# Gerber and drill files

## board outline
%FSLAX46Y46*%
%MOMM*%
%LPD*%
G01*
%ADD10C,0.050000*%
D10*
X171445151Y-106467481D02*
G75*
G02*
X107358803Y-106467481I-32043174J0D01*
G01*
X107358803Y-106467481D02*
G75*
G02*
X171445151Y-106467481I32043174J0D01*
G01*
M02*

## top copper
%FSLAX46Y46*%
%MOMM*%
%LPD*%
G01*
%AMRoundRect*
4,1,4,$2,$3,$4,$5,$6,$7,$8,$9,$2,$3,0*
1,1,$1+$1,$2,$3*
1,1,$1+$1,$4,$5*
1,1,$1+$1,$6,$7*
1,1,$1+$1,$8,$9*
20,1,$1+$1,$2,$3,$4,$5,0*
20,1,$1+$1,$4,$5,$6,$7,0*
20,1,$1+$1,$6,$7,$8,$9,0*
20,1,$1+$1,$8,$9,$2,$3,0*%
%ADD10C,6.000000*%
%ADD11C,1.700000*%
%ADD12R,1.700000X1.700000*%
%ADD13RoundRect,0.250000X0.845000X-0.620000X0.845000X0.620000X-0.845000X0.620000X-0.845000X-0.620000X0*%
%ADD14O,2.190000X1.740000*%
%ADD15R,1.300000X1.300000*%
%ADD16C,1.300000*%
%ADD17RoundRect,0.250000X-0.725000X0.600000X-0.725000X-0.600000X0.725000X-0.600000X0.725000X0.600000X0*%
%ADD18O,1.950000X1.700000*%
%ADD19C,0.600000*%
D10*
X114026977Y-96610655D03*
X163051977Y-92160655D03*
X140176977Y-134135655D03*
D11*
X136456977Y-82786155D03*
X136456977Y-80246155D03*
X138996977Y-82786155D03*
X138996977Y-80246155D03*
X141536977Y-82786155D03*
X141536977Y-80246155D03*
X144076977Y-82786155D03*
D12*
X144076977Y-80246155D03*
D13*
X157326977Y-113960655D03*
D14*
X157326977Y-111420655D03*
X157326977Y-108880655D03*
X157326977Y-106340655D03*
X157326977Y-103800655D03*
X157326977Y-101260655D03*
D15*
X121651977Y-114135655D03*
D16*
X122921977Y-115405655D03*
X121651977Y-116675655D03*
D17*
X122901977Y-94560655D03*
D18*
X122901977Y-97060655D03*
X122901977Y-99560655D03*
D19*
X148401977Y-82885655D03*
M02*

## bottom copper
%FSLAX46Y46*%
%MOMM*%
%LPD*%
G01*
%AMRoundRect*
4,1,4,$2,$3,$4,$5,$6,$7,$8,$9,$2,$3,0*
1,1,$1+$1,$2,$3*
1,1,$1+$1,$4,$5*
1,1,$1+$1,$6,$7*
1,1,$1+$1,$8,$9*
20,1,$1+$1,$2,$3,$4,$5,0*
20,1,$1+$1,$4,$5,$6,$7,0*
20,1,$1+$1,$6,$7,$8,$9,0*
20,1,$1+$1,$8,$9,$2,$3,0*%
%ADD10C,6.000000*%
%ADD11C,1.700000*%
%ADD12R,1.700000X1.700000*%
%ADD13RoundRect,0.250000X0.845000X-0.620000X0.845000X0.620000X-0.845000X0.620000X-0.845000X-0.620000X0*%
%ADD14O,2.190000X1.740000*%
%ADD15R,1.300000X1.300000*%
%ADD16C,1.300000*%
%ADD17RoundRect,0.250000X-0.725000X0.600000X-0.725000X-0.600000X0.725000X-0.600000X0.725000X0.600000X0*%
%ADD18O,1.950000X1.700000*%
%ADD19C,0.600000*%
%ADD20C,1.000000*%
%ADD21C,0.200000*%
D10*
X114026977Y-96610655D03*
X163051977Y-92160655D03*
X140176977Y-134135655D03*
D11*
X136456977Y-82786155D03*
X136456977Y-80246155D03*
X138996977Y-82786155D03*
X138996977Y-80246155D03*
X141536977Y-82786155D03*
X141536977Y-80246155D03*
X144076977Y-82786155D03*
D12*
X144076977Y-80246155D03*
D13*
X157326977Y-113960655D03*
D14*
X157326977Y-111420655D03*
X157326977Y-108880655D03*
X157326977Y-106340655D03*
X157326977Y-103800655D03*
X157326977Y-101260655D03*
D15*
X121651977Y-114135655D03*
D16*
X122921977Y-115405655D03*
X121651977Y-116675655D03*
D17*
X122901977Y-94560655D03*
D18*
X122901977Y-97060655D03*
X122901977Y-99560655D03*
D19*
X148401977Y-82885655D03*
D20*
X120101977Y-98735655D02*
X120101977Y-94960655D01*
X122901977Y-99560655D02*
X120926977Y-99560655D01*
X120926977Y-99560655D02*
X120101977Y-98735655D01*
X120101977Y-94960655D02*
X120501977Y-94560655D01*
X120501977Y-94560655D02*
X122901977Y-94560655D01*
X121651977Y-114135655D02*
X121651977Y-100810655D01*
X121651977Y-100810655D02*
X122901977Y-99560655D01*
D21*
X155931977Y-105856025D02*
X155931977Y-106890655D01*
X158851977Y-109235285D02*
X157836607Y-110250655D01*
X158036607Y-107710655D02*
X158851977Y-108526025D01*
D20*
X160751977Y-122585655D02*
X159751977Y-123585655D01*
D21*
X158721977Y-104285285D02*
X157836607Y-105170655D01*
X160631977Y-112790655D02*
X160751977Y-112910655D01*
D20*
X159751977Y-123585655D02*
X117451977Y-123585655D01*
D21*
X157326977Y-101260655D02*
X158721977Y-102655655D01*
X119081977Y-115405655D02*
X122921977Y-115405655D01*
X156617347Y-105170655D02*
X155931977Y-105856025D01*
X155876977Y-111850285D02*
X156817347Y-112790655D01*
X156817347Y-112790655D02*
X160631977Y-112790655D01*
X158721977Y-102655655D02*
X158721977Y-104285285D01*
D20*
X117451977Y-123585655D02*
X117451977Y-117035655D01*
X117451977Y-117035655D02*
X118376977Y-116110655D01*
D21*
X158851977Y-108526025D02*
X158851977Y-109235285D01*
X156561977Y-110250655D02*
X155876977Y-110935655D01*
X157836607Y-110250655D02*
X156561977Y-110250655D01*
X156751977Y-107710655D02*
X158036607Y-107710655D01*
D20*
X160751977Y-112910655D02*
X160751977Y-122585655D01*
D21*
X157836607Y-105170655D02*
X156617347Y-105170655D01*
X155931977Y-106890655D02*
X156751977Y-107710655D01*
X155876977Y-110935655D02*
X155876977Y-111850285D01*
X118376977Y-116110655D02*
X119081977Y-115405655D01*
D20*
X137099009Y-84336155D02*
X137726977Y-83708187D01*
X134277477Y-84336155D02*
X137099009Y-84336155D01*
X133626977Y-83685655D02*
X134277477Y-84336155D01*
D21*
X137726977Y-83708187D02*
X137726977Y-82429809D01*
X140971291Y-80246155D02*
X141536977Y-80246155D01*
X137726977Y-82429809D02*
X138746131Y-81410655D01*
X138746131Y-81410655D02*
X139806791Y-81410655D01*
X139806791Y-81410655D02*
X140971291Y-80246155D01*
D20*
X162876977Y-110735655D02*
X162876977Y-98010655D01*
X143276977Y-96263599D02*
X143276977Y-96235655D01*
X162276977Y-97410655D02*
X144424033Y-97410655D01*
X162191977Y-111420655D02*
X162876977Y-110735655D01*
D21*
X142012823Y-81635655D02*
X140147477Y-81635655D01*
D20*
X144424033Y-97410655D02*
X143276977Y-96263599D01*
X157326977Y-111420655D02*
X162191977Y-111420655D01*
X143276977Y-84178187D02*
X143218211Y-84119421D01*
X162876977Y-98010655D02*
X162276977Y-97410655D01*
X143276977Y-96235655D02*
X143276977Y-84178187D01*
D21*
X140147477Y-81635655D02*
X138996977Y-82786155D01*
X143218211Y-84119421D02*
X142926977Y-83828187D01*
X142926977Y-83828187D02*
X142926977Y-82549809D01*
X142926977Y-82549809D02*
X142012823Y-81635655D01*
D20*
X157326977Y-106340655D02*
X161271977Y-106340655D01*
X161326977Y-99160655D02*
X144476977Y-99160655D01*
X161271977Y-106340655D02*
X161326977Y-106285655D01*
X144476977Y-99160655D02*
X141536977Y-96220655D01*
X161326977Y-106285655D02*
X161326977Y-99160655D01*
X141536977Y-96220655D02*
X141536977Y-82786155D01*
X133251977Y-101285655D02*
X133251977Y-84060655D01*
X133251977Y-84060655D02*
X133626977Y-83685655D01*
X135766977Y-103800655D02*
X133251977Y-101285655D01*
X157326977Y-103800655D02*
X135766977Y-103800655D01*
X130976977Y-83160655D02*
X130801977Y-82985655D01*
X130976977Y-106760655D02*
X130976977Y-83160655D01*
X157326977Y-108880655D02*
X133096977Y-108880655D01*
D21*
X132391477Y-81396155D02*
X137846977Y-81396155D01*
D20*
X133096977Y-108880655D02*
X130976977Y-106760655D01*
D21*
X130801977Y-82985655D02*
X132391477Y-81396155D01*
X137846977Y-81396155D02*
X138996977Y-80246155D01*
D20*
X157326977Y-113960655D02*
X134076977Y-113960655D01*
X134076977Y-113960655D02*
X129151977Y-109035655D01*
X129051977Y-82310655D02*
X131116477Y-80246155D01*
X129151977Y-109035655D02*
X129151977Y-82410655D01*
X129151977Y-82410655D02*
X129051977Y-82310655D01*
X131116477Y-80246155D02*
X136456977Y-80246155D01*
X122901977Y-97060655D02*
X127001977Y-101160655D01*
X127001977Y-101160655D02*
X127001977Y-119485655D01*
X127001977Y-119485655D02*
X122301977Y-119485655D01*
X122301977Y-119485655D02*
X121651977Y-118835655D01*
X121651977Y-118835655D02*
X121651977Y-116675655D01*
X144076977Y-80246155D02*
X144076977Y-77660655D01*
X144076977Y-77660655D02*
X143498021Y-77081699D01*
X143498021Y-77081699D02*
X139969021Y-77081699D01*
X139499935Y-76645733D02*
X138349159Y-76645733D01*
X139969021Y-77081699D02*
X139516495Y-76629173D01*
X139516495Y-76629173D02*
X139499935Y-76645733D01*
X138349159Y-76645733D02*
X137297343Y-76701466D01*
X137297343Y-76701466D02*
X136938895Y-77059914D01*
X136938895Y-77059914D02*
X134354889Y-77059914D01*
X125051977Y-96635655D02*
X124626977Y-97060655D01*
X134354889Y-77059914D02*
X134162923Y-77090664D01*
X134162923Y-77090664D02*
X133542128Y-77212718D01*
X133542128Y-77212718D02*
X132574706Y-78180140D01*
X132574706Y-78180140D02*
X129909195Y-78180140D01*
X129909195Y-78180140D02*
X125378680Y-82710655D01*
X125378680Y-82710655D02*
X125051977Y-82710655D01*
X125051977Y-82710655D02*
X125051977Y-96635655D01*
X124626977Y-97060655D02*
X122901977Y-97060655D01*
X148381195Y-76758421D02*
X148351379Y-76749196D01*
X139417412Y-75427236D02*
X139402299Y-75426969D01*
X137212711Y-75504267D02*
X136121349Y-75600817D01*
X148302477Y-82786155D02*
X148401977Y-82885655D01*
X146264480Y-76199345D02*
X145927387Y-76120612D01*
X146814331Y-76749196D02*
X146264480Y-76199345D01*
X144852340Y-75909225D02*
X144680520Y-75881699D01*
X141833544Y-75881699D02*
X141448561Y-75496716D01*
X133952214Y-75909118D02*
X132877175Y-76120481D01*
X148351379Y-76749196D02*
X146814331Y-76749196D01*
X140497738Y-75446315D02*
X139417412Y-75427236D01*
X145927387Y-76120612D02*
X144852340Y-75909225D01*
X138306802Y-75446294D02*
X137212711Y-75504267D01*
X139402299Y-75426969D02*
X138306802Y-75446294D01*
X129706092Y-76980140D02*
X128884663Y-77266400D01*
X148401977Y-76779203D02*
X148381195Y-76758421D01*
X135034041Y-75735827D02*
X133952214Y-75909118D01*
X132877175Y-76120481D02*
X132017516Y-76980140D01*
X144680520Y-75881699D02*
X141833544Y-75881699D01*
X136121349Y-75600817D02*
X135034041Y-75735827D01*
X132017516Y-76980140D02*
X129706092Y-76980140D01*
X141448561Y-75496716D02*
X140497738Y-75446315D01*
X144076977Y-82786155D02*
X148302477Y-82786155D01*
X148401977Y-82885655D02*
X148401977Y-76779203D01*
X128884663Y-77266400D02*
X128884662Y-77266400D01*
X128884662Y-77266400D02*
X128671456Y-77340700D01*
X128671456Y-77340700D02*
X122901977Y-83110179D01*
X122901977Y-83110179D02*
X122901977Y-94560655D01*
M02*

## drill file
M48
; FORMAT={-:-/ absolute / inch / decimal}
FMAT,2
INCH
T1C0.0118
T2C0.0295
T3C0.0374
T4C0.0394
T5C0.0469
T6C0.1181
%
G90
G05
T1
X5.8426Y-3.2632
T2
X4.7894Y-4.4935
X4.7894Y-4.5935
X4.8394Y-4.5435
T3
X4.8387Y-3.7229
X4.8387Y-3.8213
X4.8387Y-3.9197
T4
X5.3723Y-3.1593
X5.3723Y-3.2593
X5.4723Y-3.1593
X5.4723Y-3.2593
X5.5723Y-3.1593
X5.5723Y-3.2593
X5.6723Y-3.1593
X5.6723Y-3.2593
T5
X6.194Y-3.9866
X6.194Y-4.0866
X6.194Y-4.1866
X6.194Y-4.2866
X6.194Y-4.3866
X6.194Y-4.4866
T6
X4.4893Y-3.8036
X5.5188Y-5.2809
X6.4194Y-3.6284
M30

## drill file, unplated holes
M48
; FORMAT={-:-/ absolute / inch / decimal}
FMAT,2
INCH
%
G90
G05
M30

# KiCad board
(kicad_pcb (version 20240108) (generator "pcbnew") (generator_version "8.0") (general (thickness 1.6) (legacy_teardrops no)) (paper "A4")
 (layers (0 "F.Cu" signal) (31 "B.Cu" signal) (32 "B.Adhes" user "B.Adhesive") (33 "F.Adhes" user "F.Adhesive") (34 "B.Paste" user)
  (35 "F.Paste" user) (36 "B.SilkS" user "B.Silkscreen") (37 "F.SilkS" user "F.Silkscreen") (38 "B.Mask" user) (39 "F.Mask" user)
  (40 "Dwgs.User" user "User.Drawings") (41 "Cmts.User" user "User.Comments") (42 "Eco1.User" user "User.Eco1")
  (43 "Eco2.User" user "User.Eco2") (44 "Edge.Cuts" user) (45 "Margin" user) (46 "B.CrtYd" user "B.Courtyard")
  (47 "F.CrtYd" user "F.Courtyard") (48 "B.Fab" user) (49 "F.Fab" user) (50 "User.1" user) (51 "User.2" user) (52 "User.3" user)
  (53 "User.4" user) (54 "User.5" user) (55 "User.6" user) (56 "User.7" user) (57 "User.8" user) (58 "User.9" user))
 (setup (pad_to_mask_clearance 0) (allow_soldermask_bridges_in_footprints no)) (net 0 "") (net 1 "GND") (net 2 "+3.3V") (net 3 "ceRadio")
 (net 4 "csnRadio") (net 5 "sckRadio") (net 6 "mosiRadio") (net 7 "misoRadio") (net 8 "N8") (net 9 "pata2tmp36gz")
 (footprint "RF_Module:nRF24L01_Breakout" (layer "F.Cu") (at 144.076977 80.246155 -90)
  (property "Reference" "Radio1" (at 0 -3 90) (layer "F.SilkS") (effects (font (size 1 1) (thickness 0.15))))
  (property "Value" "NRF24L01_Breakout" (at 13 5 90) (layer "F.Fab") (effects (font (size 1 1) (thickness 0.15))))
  (pad "1" thru_hole rect (at 0 0 270) (size 1.7 1.7) (drill 1) (layers "*.Cu" "*.Mask") (remove_unused_layers no) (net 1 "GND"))
  (pad "2" thru_hole circle (at 2.54 0 270) (size 1.7 1.7) (drill 1) (layers "*.Cu" "*.Mask") (remove_unused_layers no) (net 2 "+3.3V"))
  (pad "3" thru_hole circle (at 0 2.54 270) (size 1.7 1.7) (drill 1) (layers "*.Cu" "*.Mask") (remove_unused_layers no) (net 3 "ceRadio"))
  (pad "4" thru_hole circle (at 2.54 2.54 270) (size 1.7 1.7) (drill 1) (layers "*.Cu" "*.Mask") (remove_unused_layers no)
   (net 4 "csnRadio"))
  (pad "5" thru_hole circle (at 0 5.08 270) (size 1.7 1.7) (drill 1) (layers "*.Cu" "*.Mask") (remove_unused_layers no) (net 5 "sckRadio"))
  (pad "6" thru_hole circle (at 2.54 5.08 270) (size 1.7 1.7) (drill 1) (layers "*.Cu" "*.Mask") (remove_unused_layers no)
   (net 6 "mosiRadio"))
  (pad "7" thru_hole circle (at 0 7.62 270) (size 1.7 1.7) (drill 1) (layers "*.Cu" "*.Mask") (remove_unused_layers no) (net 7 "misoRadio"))
  (pad "8" thru_hole circle (at 2.54 7.62 270) (size 1.7 1.7) (drill 1) (layers "*.Cu" "*.Mask") (remove_unused_layers no) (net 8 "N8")))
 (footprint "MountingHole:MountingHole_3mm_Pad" (layer "F.Cu") (at 163.051977 92.160655)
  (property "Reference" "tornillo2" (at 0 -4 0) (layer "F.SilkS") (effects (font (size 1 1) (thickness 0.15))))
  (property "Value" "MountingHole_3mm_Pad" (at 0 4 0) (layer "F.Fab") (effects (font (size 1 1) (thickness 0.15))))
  (pad "2" thru_hole circle (at 0 0) (size 6 6) (drill 3) (layers "*.Cu" "*.Mask") (remove_unused_layers no)))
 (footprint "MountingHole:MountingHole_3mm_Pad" (layer "F.Cu") (at 114.026977 96.610655)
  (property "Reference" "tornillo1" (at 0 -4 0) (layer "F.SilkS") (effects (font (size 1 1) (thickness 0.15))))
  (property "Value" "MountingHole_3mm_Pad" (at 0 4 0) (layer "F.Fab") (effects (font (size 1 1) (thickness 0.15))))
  (pad "1" thru_hole circle (at 0 0) (size 6 6) (drill 3) (layers "*.Cu" "*.Mask") (remove_unused_layers no)))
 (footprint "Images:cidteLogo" (layer "F.Cu") (at 139.276977 106.160655 90)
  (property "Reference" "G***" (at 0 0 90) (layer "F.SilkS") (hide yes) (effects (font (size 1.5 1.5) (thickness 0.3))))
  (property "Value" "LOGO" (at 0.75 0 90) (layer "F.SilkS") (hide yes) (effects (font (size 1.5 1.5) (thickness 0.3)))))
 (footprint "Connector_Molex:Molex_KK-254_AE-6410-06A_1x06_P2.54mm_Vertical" (layer "F.Cu") (at 157.326977 113.960655 90)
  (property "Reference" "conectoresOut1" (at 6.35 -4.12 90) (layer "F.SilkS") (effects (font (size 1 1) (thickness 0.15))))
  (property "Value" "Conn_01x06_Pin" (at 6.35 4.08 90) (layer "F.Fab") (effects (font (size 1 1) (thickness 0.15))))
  (pad "1" thru_hole roundrect (at 0 0 90) (size 1.74 2.19) (drill 1.19) (layers "*.Cu" "*.Mask") (remove_unused_layers no)
   (roundrect_rratio 0.143678) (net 7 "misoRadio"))
  (pad "2" thru_hole oval (at 2.54 0 90) (size 1.74 2.19) (drill 1.19) (layers "*.Cu" "*.Mask") (remove_unused_layers no)
   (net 6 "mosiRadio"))
  (pad "3" thru_hole oval (at 5.08 0 90) (size 1.74 2.19) (drill 1.19) (layers "*.Cu" "*.Mask") (remove_unused_layers no) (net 5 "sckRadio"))
  (pad "4" thru_hole oval (at 7.62 0 90) (size 1.74 2.19) (drill 1.19) (layers "*.Cu" "*.Mask") (remove_unused_layers no) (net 4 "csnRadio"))
  (pad "5" thru_hole oval (at 10.16 0 90) (size 1.74 2.19) (drill 1.19) (layers "*.Cu" "*.Mask") (remove_unused_layers no) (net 3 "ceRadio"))
  (pad "6" thru_hole oval (at 12.7 0 90) (size 1.74 2.19) (drill 1.19) (layers "*.Cu" "*.Mask") (remove_unused_layers no)
   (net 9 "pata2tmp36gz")))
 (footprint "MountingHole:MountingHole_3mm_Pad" (layer "F.Cu") (at 140.176977 134.135655)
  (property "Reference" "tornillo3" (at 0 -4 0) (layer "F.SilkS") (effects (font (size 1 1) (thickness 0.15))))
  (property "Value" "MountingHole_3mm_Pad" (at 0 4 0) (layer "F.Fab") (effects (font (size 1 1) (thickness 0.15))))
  (pad "3" thru_hole circle (at 0 0) (size 6 6) (drill 3) (layers "*.Cu" "*.Mask") (remove_unused_layers no)))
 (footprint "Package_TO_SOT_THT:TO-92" (layer "F.Cu") (at 121.651977 114.135655 -90)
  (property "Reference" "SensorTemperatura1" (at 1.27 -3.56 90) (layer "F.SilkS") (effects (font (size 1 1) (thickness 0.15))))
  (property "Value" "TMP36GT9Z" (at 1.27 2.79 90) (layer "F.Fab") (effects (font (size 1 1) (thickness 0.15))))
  (pad "1" thru_hole rect (at 0 0 270) (size 1.3 1.3) (drill 0.75) (layers "*.Cu" "*.Mask") (remove_unused_layers no) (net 2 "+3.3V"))
  (pad "2" thru_hole circle (at 1.27 -1.27 270) (size 1.3 1.3) (drill 0.75) (layers "*.Cu" "*.Mask") (remove_unused_layers no)
   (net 9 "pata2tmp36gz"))
  (pad "3" thru_hole circle (at 2.54 0 270) (size 1.3 1.3) (drill 0.75) (layers "*.Cu" "*.Mask") (remove_unused_layers no) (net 1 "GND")))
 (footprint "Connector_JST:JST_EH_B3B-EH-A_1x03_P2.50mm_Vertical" (layer "F.Cu") (at 122.901977 94.560655 -90)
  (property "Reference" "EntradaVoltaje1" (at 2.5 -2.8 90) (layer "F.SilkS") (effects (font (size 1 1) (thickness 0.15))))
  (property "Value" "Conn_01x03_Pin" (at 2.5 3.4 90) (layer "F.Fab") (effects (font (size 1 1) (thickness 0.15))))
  (pad "1" thru_hole roundrect (at 0 0 270) (size 1.7 1.95) (drill 0.95) (layers "*.Cu" "*.Mask") (remove_unused_layers no)
   (roundrect_rratio 0.147059) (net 2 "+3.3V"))
  (pad "2" thru_hole oval (at 2.5 0 270) (size 1.7 1.95) (drill 0.95) (layers "*.Cu" "*.Mask") (remove_unused_layers no) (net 1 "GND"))
  (pad "3" thru_hole oval (at 5 0 270) (size 1.7 1.95) (drill 0.95) (layers "*.Cu" "*.Mask") (remove_unused_layers no) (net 2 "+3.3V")))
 (gr_circle (center 139.401977 106.467481) (end 161.451977 129.717481) (stroke (width 0.05) (type default)) (fill none) (layer "Edge.Cuts"))
 (segment (start 137.099009 84.336155) (end 137.726977 83.708187) (width 1) (layer "B.Cu") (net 3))
 (segment (start 133.251977 84.060655) (end 133.626977 83.685655) (width 1) (layer "B.Cu") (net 3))
 (segment (start 137.726977 83.708187) (end 137.726977 82.429809) (width 0.2) (layer "B.Cu") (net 3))
 (segment (start 133.251977 101.285655) (end 133.251977 84.060655) (width 1) (layer "B.Cu") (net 3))
 (segment (start 157.326977 103.800655) (end 135.766977 103.800655) (width 1) (layer "B.Cu") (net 3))
 (segment (start 140.971291 80.246155) (end 141.536977 80.246155) (width 0.2) (layer "B.Cu") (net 3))
 (segment (start 135.766977 103.800655) (end 133.251977 101.285655) (width 1) (layer "B.Cu") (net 3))
 (segment (start 133.626977 83.685655) (end 134.277477 84.336155) (width 1) (layer "B.Cu") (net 3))
 (segment (start 138.746131 81.410655) (end 139.806791 81.410655) (width 0.2) (layer "B.Cu") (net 3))
 (segment (start 134.277477 84.336155) (end 137.099009 84.336155) (width 1) (layer "B.Cu") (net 3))
 (segment (start 137.726977 82.429809) (end 138.746131 81.410655) (width 0.2) (layer "B.Cu") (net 3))
 (segment (start 139.806791 81.410655) (end 140.971291 80.246155) (width 0.2) (layer "B.Cu") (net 3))
 (segment (start 141.536977 96.220655) (end 141.536977 82.786155) (width 1) (layer "B.Cu") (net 4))
 (segment (start 161.271977 106.340655) (end 161.326977 106.285655) (width 1) (layer "B.Cu") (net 4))
 (segment (start 157.326977 106.340655) (end 161.271977 106.340655) (width 1) (layer "B.Cu") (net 4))
 (segment (start 144.476977 99.160655) (end 141.536977 96.220655) (width 1) (layer "B.Cu") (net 4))
 (segment (start 161.326977 106.285655) (end 161.326977 99.160655) (width 1) (layer "B.Cu") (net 4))
 (segment (start 161.326977 99.160655) (end 144.476977 99.160655) (width 1) (layer "B.Cu") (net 4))
 (segment (start 130.976977 106.760655) (end 130.976977 83.160655) (width 1) (layer "B.Cu") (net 5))
 (segment (start 130.801977 82.985655) (end 132.391477 81.396155) (width 0.2) (layer "B.Cu") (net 5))
 (segment (start 133.096977 108.880655) (end 130.976977 106.760655) (width 1) (layer "B.Cu") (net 5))
 (segment (start 137.846977 81.396155) (end 138.996977 80.246155) (width 0.2) (layer "B.Cu") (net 5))
 (segment (start 132.391477 81.396155) (end 137.846977 81.396155) (width 0.2) (layer "B.Cu") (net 5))
 (segment (start 157.326977 108.880655) (end 133.096977 108.880655) (width 1) (layer "B.Cu") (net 5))
 (segment (start 130.976977 83.160655) (end 130.801977 82.985655) (width 1) (layer "B.Cu") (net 5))
 (segment (start 140.147477 81.635655) (end 138.996977 82.786155) (width 0.2) (layer "B.Cu") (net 6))
 (segment (start 142.926977 82.549809) (end 142.012823 81.635655) (width 0.2) (layer "B.Cu") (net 6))
 (segment (start 143.276977 84.178187) (end 143.218211 84.119421) (width 1) (layer "B.Cu") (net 6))
 (segment (start 143.218211 84.119421) (end 142.926977 83.828187) (width 0.2) (layer "B.Cu") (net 6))
 (segment (start 143.276977 96.235655) (end 143.276977 84.178187) (width 1) (layer "B.Cu") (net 6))
 (segment (start 157.326977 111.420655) (end 162.191977 111.420655) (width 1) (layer "B.Cu") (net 6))
 (segment (start 162.191977 111.420655) (end 162.876977 110.735655) (width 1) (layer "B.Cu") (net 6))
 (segment (start 162.276977 97.410655) (end 144.424033 97.410655) (width 1) (layer "B.Cu") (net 6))
 (segment (start 162.876977 110.735655) (end 162.876977 98.010655) (width 1) (layer "B.Cu") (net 6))
 (segment (start 162.876977 98.010655) (end 162.276977 97.410655) (width 1) (layer "B.Cu") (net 6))
 (segment (start 142.012823 81.635655) (end 140.147477 81.635655) (width 0.2) (layer "B.Cu") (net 6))
 (segment (start 144.424033 97.410655) (end 143.276977 96.263599) (width 1) (layer "B.Cu") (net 6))
 (segment (start 143.276977 96.263599) (end 143.276977 96.235655) (width 1) (layer "B.Cu") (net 6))
 (segment (start 142.926977 83.828187) (end 142.926977 82.549809) (width 0.2) (layer "B.Cu") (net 6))
 (segment (start 129.151977 109.035655) (end 129.151977 82.410655) (width 1) (layer "B.Cu") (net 7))
 (segment (start 129.051977 82.310655) (end 131.116477 80.246155) (width 1) (layer "B.Cu") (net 7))
 (segment (start 129.151977 82.410655) (end 129.051977 82.310655) (width 1) (layer "B.Cu") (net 7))
 (segment (start 131.116477 80.246155) (end 136.456977 80.246155) (width 1) (layer "B.Cu") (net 7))
 (segment (start 134.076977 113.960655) (end 129.151977 109.035655) (width 1) (layer "B.Cu") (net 7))
 (segment (start 157.326977 113.960655) (end 134.076977 113.960655) (width 1) (layer "B.Cu") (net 7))
 (segment (start 160.751977 122.585655) (end 159.751977 123.585655) (width 1) (layer "B.Cu") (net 9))
 (segment (start 160.631977 112.790655) (end 160.751977 112.910655) (width 0.2) (layer "B.Cu") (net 9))
 (segment (start 160.751977 112.910655) (end 160.751977 122.585655) (width 1) (layer "B.Cu") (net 9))
 (segment (start 155.876977 110.935655) (end 155.876977 111.850285) (width 0.2) (layer "B.Cu") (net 9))
 (segment (start 155.931977 106.890655) (end 156.751977 107.710655) (width 0.2) (layer "B.Cu") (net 9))
 (segment (start 156.751977 107.710655) (end 158.036607 107.710655) (width 0.2) (layer "B.Cu") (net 9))
 (segment (start 159.751977 123.585655) (end 117.451977 123.585655) (width 1) (layer "B.Cu") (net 9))
 (segment (start 158.721977 102.655655) (end 158.721977 104.285285) (width 0.2) (layer "B.Cu") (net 9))
 (segment (start 158.036607 107.710655) (end 158.851977 108.526025) (width 0.2) (layer "B.Cu") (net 9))
 (segment (start 157.836607 105.170655) (end 156.617347 105.170655) (width 0.2) (layer "B.Cu") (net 9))
 (segment (start 155.876977 111.850285) (end 156.817347 112.790655) (width 0.2) (layer "B.Cu") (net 9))
 (segment (start 158.851977 109.235285) (end 157.836607 110.250655) (width 0.2) (layer "B.Cu") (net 9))
 (segment (start 156.817347 112.790655) (end 160.631977 112.790655) (width 0.2) (layer "B.Cu") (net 9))
 (segment (start 158.851977 108.526025) (end 158.851977 109.235285) (width 0.2) (layer "B.Cu") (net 9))
 (segment (start 117.451977 117.035655) (end 118.376977 116.110655) (width 1) (layer "B.Cu") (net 9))
 (segment (start 156.561977 110.250655) (end 155.876977 110.935655) (width 0.2) (layer "B.Cu") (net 9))
 (segment (start 158.721977 104.285285) (end 157.836607 105.170655) (width 0.2) (layer "B.Cu") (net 9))
 (segment (start 118.376977 116.110655) (end 119.081977 115.405655) (width 0.2) (layer "B.Cu") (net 9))
 (segment (start 155.931977 105.856025) (end 155.931977 106.890655) (width 0.2) (layer "B.Cu") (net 9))
 (segment (start 117.451977 123.585655) (end 117.451977 117.035655) (width 1) (layer "B.Cu") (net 9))
 (segment (start 157.326977 101.260655) (end 158.721977 102.655655) (width 0.2) (layer "B.Cu") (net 9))
 (segment (start 156.617347 105.170655) (end 155.931977 105.856025) (width 0.2) (layer "B.Cu") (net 9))
 (segment (start 157.836607 110.250655) (end 156.561977 110.250655) (width 0.2) (layer "B.Cu") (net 9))
 (segment (start 119.081977 115.405655) (end 122.921977 115.405655) (width 0.2) (layer "B.Cu") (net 9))
 (via (at 148.401977 82.885655) (size 0.6) (drill 0.3) (layers "F.Cu" "B.Cu") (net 2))
 (segment (start 144.85234 75.909225) (end 144.68052 75.881699) (width 1) (layer "B.Cu") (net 2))
 (segment (start 133.952214 75.909118) (end 132.877175 76.120481) (width 1) (layer "B.Cu") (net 2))
 (segment (start 122.901977 99.560655) (end 120.926977 99.560655) (width 1) (layer "B.Cu") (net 2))
 (segment (start 120.926977 99.560655) (end 120.101977 98.735655) (width 1) (layer "B.Cu") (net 2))
 (segment (start 148.381195 76.758421) (end 148.351379 76.749196) (width 1) (layer "B.Cu") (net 2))
 (segment (start 129.706092 76.98014) (end 128.884663 77.2664) (width 1) (layer "B.Cu") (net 2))
 (segment (start 120.101977 98.735655) (end 120.101977 94.960655) (width 1) (layer "B.Cu") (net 2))
 (segment (start 137.212711 75.504267) (end 136.121349 75.600817) (width 1) (layer "B.Cu") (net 2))
 (segment (start 144.68052 75.881699) (end 141.833544 75.881699) (width 1) (layer "B.Cu") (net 2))
 (segment (start 148.302477 82.786155) (end 148.401977 82.885655) (width 1) (layer "B.Cu") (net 2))
 (segment (start 148.351379 76.749196) (end 146.814331 76.749196) (width 1) (layer "B.Cu") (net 2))
 (segment (start 132.017516 76.98014) (end 129.706092 76.98014) (width 1) (layer "B.Cu") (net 2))
 (segment (start 141.833544 75.881699) (end 141.448561 75.496716) (width 1) (layer "B.Cu") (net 2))
 (segment (start 128.671456 77.3407) (end 122.901977 83.110179) (width 1) (layer "B.Cu") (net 2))
 (segment (start 135.034041 75.735827) (end 133.952214 75.909118) (width 1) (layer "B.Cu") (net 2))
 (segment (start 148.401977 82.885655) (end 148.401977 76.779203) (width 1) (layer "B.Cu") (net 2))
 (segment (start 148.401977 76.779203) (end 148.381195 76.758421) (width 1) (layer "B.Cu") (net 2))
 (segment (start 121.651977 114.135655) (end 121.651977 100.810655) (width 1) (layer "B.Cu") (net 2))
 (segment (start 141.448561 75.496716) (end 140.497738 75.446315) (width 1) (layer "B.Cu") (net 2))
 (segment (start 128.884663 77.2664) (end 128.884662 77.2664) (width 1) (layer "B.Cu") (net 2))
 (segment (start 139.417412 75.427236) (end 139.402299 75.426969) (width 1) (layer "B.Cu") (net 2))
 (segment (start 132.877175 76.120481) (end 132.017516 76.98014) (width 1) (layer "B.Cu") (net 2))
 (segment (start 128.884662 77.2664) (end 128.671456 77.3407) (width 1) (layer "B.Cu") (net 2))
 (segment (start 140.497738 75.446315) (end 139.417412 75.427236) (width 1) (layer "B.Cu") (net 2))
 (segment (start 138.306802 75.446294) (end 137.212711 75.504267) (width 1) (layer "B.Cu") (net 2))
 (segment (start 121.651977 100.810655) (end 122.901977 99.560655) (width 1) (layer "B.Cu") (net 2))
 (segment (start 144.076977 82.786155) (end 148.302477 82.786155) (width 1) (layer "B.Cu") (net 2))
 (segment (start 145.927387 76.120612) (end 144.85234 75.909225) (width 1) (layer "B.Cu") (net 2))
 (segment (start 120.501977 94.560655) (end 122.901977 94.560655) (width 1) (layer "B.Cu") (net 2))
 (segment (start 139.402299 75.426969) (end 138.306802 75.446294) (width 1) (layer "B.Cu") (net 2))
 (segment (start 146.814331 76.749196) (end 146.26448 76.199345) (width 1) (layer "B.Cu") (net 2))
 (segment (start 120.101977 94.960655) (end 120.501977 94.560655) (width 1) (layer "B.Cu") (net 2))
 (segment (start 136.121349 75.600817) (end 135.034041 75.735827) (width 1) (layer "B.Cu") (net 2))
 (segment (start 146.26448 76.199345) (end 145.927387 76.120612) (width 1) (layer "B.Cu") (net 2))
 (segment (start 122.901977 83.110179) (end 122.901977 94.560655) (width 1) (layer "B.Cu") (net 2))
 (segment (start 124.626977 97.060655) (end 122.901977 97.060655) (width 1) (layer "B.Cu") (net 1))
 (segment (start 121.651977 118.835655) (end 121.651977 116.675655) (width 1) (layer "B.Cu") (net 1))
 (segment (start 125.051977 82.710655) (end 125.051977 96.635655) (width 1) (layer "B.Cu") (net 1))
 (segment (start 134.354889 77.059914) (end 134.162923 77.090664) (width 1) (layer "B.Cu") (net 1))
 (segment (start 122.901977 97.060655) (end 127.001977 101.160655) (width 1) (layer "B.Cu") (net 1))
 (segment (start 139.516495 76.629173) (end 139.499935 76.645733) (width 1) (layer "B.Cu") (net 1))
 (segment (start 134.162923 77.090664) (end 133.542128 77.212718) (width 1) (layer "B.Cu") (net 1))
 (segment (start 139.969021 77.081699) (end 139.516495 76.629173) (width 1) (layer "B.Cu") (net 1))
 (segment (start 136.938895 77.059914) (end 134.354889 77.059914) (width 1) (layer "B.Cu") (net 1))
 (segment (start 127.001977 119.485655) (end 122.301977 119.485655) (width 1) (layer "B.Cu") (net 1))
 (segment (start 132.574706 78.18014) (end 129.909195 78.18014) (width 1) (layer "B.Cu") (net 1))
 (segment (start 144.076977 80.246155) (end 144.076977 77.660655) (width 1) (layer "B.Cu") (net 1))
 (segment (start 125.37868 82.710655) (end 125.051977 82.710655) (width 1) (layer "B.Cu") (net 1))
 (segment (start 139.499935 76.645733) (end 138.349159 76.645733) (width 1) (layer "B.Cu") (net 1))
 (segment (start 129.909195 78.18014) (end 125.37868 82.710655) (width 1) (layer "B.Cu") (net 1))
 (segment (start 127.001977 101.160655) (end 127.001977 119.485655) (width 1) (layer "B.Cu") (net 1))
 (segment (start 122.301977 119.485655) (end 121.651977 118.835655) (width 1) (layer "B.Cu") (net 1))
 (segment (start 138.349159 76.645733) (end 137.297343 76.701466) (width 1) (layer "B.Cu") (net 1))
 (segment (start 144.076977 77.660655) (end 143.498021 77.081699) (width 1) (layer "B.Cu") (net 1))
 (segment (start 125.051977 96.635655) (end 124.626977 97.060655) (width 1) (layer "B.Cu") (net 1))
 (segment (start 133.542128 77.212718) (end 132.574706 78.18014) (width 1) (layer "B.Cu") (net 1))
 (segment (start 143.498021 77.081699) (end 139.969021 77.081699) (width 1) (layer "B.Cu") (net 1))
 (segment (start 137.297343 76.701466) (end 136.938895 77.059914) (width 1) (layer "B.Cu") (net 1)))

